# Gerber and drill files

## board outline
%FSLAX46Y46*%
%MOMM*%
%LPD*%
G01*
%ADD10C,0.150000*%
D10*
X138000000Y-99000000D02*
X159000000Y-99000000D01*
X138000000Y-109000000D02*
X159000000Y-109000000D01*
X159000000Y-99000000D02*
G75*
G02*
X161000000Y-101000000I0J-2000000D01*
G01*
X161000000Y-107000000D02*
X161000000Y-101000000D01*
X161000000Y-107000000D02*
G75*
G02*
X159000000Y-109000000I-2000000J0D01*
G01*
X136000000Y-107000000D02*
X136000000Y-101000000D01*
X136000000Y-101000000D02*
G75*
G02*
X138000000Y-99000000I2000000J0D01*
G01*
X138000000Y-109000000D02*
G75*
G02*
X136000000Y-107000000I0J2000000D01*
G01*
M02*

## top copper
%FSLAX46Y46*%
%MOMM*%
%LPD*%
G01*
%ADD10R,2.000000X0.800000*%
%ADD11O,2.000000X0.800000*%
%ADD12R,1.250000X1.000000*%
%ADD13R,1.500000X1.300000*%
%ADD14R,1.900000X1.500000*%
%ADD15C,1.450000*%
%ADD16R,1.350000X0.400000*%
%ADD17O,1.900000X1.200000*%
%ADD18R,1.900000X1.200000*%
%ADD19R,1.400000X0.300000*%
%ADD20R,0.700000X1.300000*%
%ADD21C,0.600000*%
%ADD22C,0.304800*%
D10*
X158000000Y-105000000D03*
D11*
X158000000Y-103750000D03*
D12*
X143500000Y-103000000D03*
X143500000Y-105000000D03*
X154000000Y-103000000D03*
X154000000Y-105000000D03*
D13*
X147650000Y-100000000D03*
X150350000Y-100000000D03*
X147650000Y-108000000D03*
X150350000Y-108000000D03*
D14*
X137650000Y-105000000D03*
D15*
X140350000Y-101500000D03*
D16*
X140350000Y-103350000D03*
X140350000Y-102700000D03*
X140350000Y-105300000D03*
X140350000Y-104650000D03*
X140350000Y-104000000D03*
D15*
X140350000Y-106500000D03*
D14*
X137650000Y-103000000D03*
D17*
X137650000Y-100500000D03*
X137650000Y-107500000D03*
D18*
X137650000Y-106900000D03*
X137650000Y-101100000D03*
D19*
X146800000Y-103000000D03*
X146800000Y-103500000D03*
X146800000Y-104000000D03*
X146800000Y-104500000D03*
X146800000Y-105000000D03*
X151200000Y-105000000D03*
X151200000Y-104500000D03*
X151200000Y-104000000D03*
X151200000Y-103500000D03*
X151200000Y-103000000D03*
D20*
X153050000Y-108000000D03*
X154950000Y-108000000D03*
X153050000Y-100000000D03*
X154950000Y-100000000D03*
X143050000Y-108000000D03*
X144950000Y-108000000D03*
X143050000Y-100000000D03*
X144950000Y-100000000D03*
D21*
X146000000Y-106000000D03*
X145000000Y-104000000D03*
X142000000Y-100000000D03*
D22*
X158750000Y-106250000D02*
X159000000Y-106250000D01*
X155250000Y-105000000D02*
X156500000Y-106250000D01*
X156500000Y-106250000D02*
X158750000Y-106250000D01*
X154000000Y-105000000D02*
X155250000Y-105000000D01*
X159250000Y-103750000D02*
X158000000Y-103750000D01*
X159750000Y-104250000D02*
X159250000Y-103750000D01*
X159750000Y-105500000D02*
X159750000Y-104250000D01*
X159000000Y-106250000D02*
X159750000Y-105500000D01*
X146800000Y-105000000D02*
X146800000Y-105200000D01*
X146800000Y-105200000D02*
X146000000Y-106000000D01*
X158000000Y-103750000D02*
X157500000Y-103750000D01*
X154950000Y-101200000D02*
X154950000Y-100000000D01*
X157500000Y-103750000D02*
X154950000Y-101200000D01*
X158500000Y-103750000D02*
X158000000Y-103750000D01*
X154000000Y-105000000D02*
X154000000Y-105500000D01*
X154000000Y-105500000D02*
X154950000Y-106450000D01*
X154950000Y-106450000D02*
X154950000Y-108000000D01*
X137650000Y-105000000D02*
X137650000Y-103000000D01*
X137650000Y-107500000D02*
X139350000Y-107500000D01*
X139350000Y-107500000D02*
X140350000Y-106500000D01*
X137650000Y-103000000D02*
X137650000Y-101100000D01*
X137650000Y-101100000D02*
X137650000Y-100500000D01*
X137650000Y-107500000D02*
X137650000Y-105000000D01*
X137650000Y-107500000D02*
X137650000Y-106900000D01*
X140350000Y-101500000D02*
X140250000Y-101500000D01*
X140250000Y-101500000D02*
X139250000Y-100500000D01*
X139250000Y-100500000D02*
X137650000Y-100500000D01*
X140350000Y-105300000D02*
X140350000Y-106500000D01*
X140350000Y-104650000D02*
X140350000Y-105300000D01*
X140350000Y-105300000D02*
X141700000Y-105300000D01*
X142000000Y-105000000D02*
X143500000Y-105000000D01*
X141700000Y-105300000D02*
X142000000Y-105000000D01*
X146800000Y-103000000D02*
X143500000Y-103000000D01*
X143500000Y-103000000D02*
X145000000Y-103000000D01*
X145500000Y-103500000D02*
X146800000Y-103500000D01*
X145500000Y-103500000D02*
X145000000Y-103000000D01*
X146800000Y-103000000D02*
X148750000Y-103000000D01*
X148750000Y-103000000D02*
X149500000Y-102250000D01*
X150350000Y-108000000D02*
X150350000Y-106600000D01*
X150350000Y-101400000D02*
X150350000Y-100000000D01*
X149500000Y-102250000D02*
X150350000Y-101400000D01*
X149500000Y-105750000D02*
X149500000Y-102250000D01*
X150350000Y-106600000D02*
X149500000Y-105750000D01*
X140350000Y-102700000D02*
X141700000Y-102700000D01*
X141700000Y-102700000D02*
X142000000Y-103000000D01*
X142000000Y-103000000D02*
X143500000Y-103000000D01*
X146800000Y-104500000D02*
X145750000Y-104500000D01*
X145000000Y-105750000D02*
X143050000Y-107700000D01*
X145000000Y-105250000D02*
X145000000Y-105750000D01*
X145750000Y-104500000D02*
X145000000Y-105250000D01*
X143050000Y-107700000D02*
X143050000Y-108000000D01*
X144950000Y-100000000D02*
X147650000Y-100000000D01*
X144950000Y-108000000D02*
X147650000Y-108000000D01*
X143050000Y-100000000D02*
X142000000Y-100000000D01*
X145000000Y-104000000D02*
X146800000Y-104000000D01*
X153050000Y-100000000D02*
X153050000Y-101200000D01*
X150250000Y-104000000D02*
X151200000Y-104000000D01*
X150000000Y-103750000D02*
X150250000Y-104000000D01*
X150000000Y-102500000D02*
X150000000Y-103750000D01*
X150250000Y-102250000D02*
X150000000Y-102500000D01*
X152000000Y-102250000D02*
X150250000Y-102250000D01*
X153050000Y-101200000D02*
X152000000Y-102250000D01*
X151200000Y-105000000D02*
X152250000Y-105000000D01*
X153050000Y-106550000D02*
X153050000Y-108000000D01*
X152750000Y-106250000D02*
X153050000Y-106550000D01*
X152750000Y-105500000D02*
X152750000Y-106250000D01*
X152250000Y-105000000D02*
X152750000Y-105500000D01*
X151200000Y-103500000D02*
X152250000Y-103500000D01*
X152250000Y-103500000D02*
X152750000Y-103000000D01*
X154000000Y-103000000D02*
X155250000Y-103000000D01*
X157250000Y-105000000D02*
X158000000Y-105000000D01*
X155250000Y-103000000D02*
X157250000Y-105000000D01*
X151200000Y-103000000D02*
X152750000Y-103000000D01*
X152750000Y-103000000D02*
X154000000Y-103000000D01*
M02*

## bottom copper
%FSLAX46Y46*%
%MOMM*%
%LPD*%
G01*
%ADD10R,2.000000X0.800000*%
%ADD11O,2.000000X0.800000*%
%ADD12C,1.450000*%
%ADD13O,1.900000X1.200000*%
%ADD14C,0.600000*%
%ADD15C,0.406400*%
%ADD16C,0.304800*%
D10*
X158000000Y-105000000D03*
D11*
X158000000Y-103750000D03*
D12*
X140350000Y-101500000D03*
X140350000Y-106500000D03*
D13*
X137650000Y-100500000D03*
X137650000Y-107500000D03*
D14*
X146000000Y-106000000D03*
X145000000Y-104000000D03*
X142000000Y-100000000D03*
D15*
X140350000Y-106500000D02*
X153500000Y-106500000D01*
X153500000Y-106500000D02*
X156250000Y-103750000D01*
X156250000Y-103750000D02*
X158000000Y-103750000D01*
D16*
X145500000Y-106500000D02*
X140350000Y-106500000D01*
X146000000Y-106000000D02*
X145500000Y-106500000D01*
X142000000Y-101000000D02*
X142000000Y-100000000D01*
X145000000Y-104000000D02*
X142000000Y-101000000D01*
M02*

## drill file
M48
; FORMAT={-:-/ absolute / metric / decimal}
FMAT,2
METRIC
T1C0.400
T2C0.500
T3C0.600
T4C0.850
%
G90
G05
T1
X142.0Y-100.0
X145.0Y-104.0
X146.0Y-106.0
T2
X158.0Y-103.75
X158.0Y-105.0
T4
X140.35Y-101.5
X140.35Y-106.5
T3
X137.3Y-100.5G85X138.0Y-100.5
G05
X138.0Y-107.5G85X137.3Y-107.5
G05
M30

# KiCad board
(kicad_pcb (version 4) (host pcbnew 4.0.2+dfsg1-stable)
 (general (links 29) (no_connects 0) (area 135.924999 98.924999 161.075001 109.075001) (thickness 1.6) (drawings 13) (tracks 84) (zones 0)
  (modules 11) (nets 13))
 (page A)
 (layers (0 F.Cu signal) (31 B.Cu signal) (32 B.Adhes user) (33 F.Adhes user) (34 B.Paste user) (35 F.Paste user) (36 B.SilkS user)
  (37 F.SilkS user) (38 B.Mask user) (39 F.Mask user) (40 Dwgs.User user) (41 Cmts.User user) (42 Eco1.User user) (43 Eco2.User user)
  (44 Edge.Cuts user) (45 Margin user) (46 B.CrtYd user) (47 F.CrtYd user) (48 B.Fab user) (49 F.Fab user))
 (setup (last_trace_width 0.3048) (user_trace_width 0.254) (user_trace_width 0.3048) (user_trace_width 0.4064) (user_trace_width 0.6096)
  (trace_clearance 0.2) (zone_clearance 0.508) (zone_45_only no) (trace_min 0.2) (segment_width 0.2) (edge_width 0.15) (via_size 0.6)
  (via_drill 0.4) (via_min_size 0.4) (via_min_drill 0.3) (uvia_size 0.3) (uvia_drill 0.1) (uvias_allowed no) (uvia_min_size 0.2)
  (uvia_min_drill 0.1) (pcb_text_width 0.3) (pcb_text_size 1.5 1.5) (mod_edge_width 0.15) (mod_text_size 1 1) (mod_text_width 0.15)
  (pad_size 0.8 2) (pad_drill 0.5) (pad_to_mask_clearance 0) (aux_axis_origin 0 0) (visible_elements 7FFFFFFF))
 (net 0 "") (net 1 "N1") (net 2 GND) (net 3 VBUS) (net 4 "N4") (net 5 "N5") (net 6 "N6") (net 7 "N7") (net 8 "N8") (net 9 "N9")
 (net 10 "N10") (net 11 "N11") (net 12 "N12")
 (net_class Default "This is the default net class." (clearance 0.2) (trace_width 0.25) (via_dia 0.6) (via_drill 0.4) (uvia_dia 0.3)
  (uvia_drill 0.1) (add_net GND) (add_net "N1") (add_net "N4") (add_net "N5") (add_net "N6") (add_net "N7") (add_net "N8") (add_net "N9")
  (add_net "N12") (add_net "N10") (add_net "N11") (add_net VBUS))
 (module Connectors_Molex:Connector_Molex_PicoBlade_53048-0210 (layer F.Cu) (at 158 105 90)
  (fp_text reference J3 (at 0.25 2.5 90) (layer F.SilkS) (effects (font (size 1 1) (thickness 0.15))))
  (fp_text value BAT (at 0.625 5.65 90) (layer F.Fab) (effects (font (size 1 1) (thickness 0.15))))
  (pad 1 thru_hole rect (at 0 0 90) (size 0.8 2) (drill 0.5) (layers *.Cu *.Mask F.SilkS) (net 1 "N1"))
  (pad 2 thru_hole oval (at 1.25 0 90) (size 0.8 2) (drill 0.5) (layers *.Cu *.Mask F.SilkS) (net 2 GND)))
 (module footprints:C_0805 (layer F.Cu) (at 143.5 104 270)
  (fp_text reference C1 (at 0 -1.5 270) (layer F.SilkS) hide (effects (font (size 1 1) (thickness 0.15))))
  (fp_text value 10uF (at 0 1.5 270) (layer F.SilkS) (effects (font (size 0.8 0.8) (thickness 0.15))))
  (pad 1 smd rect (at -1 0 270) (size 1 1.25) (layers F.Cu F.Paste F.Mask) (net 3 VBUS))
  (pad 2 smd rect (at 1 0 270) (size 1 1.25) (layers F.Cu F.Paste F.Mask) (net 2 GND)))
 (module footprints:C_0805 (layer F.Cu) (at 154 104 270)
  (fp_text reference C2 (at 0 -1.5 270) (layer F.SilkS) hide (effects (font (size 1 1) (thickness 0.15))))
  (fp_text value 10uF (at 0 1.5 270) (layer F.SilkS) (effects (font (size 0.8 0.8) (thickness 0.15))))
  (pad 1 smd rect (at -1 0 270) (size 1 1.25) (layers F.Cu F.Paste F.Mask) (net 1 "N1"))
  (pad 2 smd rect (at 1 0 270) (size 1 1.25) (layers F.Cu F.Paste F.Mask) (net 2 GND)))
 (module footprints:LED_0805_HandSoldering (layer F.Cu) (at 149 100)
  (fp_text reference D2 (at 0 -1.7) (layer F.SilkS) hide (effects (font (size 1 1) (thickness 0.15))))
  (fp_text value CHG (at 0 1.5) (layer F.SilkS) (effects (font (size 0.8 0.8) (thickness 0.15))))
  (pad 1 smd rect (at -1.35 0) (size 1.5 1.3) (layers F.Cu F.Paste F.Mask) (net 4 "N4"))
  (pad 2 smd rect (at 1.35 0) (size 1.5 1.3) (layers F.Cu F.Paste F.Mask) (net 3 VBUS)))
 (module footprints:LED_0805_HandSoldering (layer F.Cu) (at 149 108)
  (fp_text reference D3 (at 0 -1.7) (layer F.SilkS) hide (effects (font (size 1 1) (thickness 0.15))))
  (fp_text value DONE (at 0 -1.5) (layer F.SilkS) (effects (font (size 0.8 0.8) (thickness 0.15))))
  (pad 1 smd rect (at -1.35 0) (size 1.5 1.3) (layers F.Cu F.Paste F.Mask) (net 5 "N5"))
  (pad 2 smd rect (at 1.35 0) (size 1.5 1.3) (layers F.Cu F.Paste F.Mask) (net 3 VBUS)))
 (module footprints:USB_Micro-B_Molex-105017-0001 (layer F.Cu) (at 138 104 270)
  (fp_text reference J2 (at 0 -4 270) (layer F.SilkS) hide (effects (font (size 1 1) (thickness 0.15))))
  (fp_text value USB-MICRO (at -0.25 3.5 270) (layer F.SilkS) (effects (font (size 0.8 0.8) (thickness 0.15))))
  (pad 5 smd rect (at 1 0.35 270) (size 1.5 1.9) (layers F.Cu F.Paste F.Mask) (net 2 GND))
  (pad 5 thru_hole circle (at -2.5 -2.35 270) (size 1.45 1.45) (drill 0.85) (layers *.Cu *.Mask) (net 2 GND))
  (pad 2 smd rect (at -0.65 -2.35 270) (size 0.4 1.35) (layers F.Cu F.Paste F.Mask) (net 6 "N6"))
  (pad 1 smd rect (at -1.3 -2.35 270) (size 0.4 1.35) (layers F.Cu F.Paste F.Mask) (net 3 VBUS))
  (pad 5 smd rect (at 1.3 -2.35 270) (size 0.4 1.35) (layers F.Cu F.Paste F.Mask) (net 2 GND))
  (pad 4 smd rect (at 0.65 -2.35 270) (size 0.4 1.35) (layers F.Cu F.Paste F.Mask) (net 2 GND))
  (pad 3 smd rect (at 0 -2.35 270) (size 0.4 1.35) (layers F.Cu F.Paste F.Mask) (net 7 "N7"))
  (pad 5 thru_hole circle (at 2.5 -2.35 270) (size 1.45 1.45) (drill 0.85) (layers *.Cu *.Mask) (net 2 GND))
  (pad 5 smd rect (at -1 0.35 270) (size 1.5 1.9) (layers F.Cu F.Paste F.Mask) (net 2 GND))
  (pad 5 thru_hole oval (at -3.5 0.35 90) (size 1.2 1.9) (drill oval 0.6 1.3) (layers *.Cu *.Mask) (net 2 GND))
  (pad 5 thru_hole oval (at 3.5 0.35 270) (size 1.2 1.9) (drill oval 0.6 1.3) (layers *.Cu *.Mask) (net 2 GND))
  (pad 5 smd rect (at 2.9 0.35 270) (size 1.2 1.9) (layers F.Cu F.Mask) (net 2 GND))
  (pad 5 smd rect (at -2.9 0.35 270) (size 1.2 1.9) (layers F.Cu F.Mask) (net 2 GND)))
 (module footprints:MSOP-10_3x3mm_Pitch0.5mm (layer F.Cu) (at 149 104)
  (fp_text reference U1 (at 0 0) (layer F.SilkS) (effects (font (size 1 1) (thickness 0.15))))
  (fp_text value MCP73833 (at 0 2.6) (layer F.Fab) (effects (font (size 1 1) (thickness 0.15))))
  (pad 1 smd rect (at -2.2 -1) (size 1.4 0.3) (layers F.Cu F.Paste F.Mask) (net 3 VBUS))
  (pad 2 smd rect (at -2.2 -0.5) (size 1.4 0.3) (layers F.Cu F.Paste F.Mask) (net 3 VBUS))
  (pad 3 smd rect (at -2.2 0) (size 1.4 0.3) (layers F.Cu F.Paste F.Mask) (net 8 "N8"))
  (pad 4 smd rect (at -2.2 0.5) (size 1.4 0.3) (layers F.Cu F.Paste F.Mask) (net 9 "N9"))
  (pad 5 smd rect (at -2.2 1) (size 1.4 0.3) (layers F.Cu F.Paste F.Mask) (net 2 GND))
  (pad 6 smd rect (at 2.2 1) (size 1.4 0.3) (layers F.Cu F.Paste F.Mask) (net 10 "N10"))
  (pad 7 smd rect (at 2.2 0.5) (size 1.4 0.3) (layers F.Cu F.Paste F.Mask) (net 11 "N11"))
  (pad 8 smd rect (at 2.2 0) (size 1.4 0.3) (layers F.Cu F.Paste F.Mask) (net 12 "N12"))
  (pad 9 smd rect (at 2.2 -0.5) (size 1.4 0.3) (layers F.Cu F.Paste F.Mask) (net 1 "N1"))
  (pad 10 smd rect (at 2.2 -1) (size 1.4 0.3) (layers F.Cu F.Paste F.Mask) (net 1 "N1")))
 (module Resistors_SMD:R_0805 (layer F.Cu) (at 154 108)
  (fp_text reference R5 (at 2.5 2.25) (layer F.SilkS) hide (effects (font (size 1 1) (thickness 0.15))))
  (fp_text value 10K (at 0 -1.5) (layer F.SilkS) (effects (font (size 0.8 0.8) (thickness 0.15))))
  (pad 1 smd rect (at -0.95 0) (size 0.7 1.3) (layers F.Cu F.Paste F.Mask) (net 10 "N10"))
  (pad 2 smd rect (at 0.95 0) (size 0.7 1.3) (layers F.Cu F.Paste F.Mask) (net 2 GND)))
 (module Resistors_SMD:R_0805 (layer F.Cu) (at 154 100)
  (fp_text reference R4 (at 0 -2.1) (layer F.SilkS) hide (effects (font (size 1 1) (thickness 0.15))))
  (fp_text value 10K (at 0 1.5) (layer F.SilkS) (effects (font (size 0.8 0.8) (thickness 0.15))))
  (pad 1 smd rect (at -0.95 0) (size 0.7 1.3) (layers F.Cu F.Paste F.Mask) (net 12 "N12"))
  (pad 2 smd rect (at 0.95 0) (size 0.7 1.3) (layers F.Cu F.Paste F.Mask) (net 2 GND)))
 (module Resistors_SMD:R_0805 (layer F.Cu) (at 144 108)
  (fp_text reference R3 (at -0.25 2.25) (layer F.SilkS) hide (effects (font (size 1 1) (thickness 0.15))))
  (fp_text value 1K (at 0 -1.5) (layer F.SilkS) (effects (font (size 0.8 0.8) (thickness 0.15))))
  (pad 1 smd rect (at -0.95 0) (size 0.7 1.3) (layers F.Cu F.Paste F.Mask) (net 9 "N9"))
  (pad 2 smd rect (at 0.95 0) (size 0.7 1.3) (layers F.Cu F.Paste F.Mask) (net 5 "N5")))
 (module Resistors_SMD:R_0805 (layer F.Cu) (at 144 100)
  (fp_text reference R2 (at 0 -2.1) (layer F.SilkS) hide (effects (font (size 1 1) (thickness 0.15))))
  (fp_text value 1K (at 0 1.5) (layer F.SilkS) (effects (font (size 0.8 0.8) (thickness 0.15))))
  (pad 1 smd rect (at -0.95 0) (size 0.7 1.3) (layers F.Cu F.Paste F.Mask) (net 8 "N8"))
  (pad 2 smd rect (at 0.95 0) (size 0.7 1.3) (layers F.Cu F.Paste F.Mask) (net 4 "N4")))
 (gr_line (start 138 99) (end 159 99) (angle 90) (layer Edge.Cuts) (width 0.15))
 (gr_line (start 138 109) (end 159 109) (angle 90) (layer Edge.Cuts) (width 0.15))
 (gr_arc (start 159 101) (end 159 99) (angle 90) (layer Edge.Cuts) (width 0.15))
 (gr_line (start 161 107) (end 161 101) (angle 90) (layer Edge.Cuts) (width 0.15))
 (gr_arc (start 159 107) (end 161 107) (angle 90) (layer Edge.Cuts) (width 0.15))
 (gr_line (start 136 107) (end 136 101) (angle 90) (layer Edge.Cuts) (width 0.15))
 (gr_arc (start 138 101) (end 136 101) (angle 90) (layer Edge.Cuts) (width 0.15))
 (gr_arc (start 138 107) (end 138 109) (angle 90) (layer Edge.Cuts) (width 0.15))
 (segment (start 158.75 106.25) (end 159 106.25) (width 0.3048) (layer F.Cu) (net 2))
 (segment (start 155.25 105) (end 156.5 106.25) (width 0.3048) (layer F.Cu) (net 2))
 (segment (start 156.5 106.25) (end 158.75 106.25) (width 0.3048) (layer F.Cu) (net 2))
 (segment (start 154 105) (end 155.25 105) (width 0.3048) (layer F.Cu) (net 2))
 (segment (start 159.25 103.75) (end 158 103.75) (width 0.3048) (layer F.Cu) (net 2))
 (segment (start 159.75 104.25) (end 159.25 103.75) (width 0.3048) (layer F.Cu) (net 2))
 (segment (start 159.75 105.5) (end 159.75 104.25) (width 0.3048) (layer F.Cu) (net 2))
 (segment (start 159 106.25) (end 159.75 105.5) (width 0.3048) (layer F.Cu) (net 2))
 (segment (start 140.35 106.5) (end 153.5 106.5) (width 0.4064) (layer B.Cu) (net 2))
 (segment (start 153.5 106.5) (end 156.25 103.75) (width 0.4064) (layer B.Cu) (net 2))
 (segment (start 156.25 103.75) (end 158 103.75) (width 0.4064) (layer B.Cu) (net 2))
 (segment (start 146.8 105) (end 146.8 105.2) (width 0.3048) (layer F.Cu) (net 2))
 (segment (start 145.5 106.5) (end 140.35 106.5) (width 0.3048) (layer B.Cu) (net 2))
 (segment (start 146 106) (end 145.5 106.5) (width 0.3048) (layer B.Cu) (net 2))
 (via (at 146 106) (size 0.6) (drill 0.4) (layers F.Cu B.Cu) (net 2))
 (segment (start 146.8 105.2) (end 146 106) (width 0.3048) (layer F.Cu) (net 2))
 (segment (start 158 103.75) (end 157.5 103.75) (width 0.3048) (layer F.Cu) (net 2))
 (segment (start 154.95 101.2) (end 154.95 100) (width 0.3048) (layer F.Cu) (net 2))
 (segment (start 157.5 103.75) (end 154.95 101.2) (width 0.3048) (layer F.Cu) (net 2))
 (segment (start 158.5 103.75) (end 158 103.75) (width 0.3048) (layer F.Cu) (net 2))
 (segment (start 154 105) (end 154 105.5) (width 0.3048) (layer F.Cu) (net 2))
 (segment (start 154 105.5) (end 154.95 106.45) (width 0.3048) (layer F.Cu) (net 2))
 (segment (start 154.95 106.45) (end 154.95 108) (width 0.3048) (layer F.Cu) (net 2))
 (segment (start 137.65 105) (end 137.65 103) (width 0.3048) (layer F.Cu) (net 2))
 (segment (start 137.65 107.5) (end 139.35 107.5) (width 0.3048) (layer F.Cu) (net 2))
 (segment (start 139.35 107.5) (end 140.35 106.5) (width 0.3048) (layer F.Cu) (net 2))
 (segment (start 137.65 103) (end 137.65 101.1) (width 0.3048) (layer F.Cu) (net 2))
 (segment (start 137.65 101.1) (end 137.65 100.5) (width 0.3048) (layer F.Cu) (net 2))
 (segment (start 137.65 107.5) (end 137.65 105) (width 0.3048) (layer F.Cu) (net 2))
 (segment (start 137.65 107.5) (end 137.65 106.9) (width 0.3048) (layer F.Cu) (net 2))
 (segment (start 140.35 101.5) (end 140.25 101.5) (width 0.3048) (layer F.Cu) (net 2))
 (segment (start 140.25 101.5) (end 139.25 100.5) (width 0.3048) (layer F.Cu) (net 2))
 (segment (start 139.25 100.5) (end 137.65 100.5) (width 0.3048) (layer F.Cu) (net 2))
 (segment (start 140.35 105.3) (end 140.35 106.5) (width 0.3048) (layer F.Cu) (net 2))
 (segment (start 140.35 104.65) (end 140.35 105.3) (width 0.3048) (layer F.Cu) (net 2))
 (segment (start 140.35 105.3) (end 141.7 105.3) (width 0.3048) (layer F.Cu) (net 2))
 (segment (start 142 105) (end 143.5 105) (width 0.3048) (layer F.Cu) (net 2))
 (segment (start 141.7 105.3) (end 142 105) (width 0.3048) (layer F.Cu) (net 2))
 (segment (start 146.8 103) (end 143.5 103) (width 0.3048) (layer F.Cu) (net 3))
 (segment (start 143.5 103) (end 145 103) (width 0.3048) (layer F.Cu) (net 3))
 (segment (start 145.5 103.5) (end 146.8 103.5) (width 0.3048) (layer F.Cu) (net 3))
 (segment (start 145.5 103.5) (end 145 103) (width 0.3048) (layer F.Cu) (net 3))
 (segment (start 146.8 103) (end 148.75 103) (width 0.3048) (layer F.Cu) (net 3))
 (segment (start 148.75 103) (end 149.5 102.25) (width 0.3048) (layer F.Cu) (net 3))
 (segment (start 150.35 108) (end 150.35 106.6) (width 0.3048) (layer F.Cu) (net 3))
 (segment (start 150.35 101.4) (end 150.35 100) (width 0.3048) (layer F.Cu) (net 3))
 (segment (start 149.5 102.25) (end 150.35 101.4) (width 0.3048) (layer F.Cu) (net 3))
 (segment (start 149.5 105.75) (end 149.5 102.25) (width 0.3048) (layer F.Cu) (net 3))
 (segment (start 150.35 106.6) (end 149.5 105.75) (width 0.3048) (layer F.Cu) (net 3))
 (segment (start 140.35 102.7) (end 141.7 102.7) (width 0.3048) (layer F.Cu) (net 3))
 (segment (start 141.7 102.7) (end 142 103) (width 0.3048) (layer F.Cu) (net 3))
 (segment (start 142 103) (end 143.5 103) (width 0.3048) (layer F.Cu) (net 3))
 (segment (start 146.8 104.5) (end 145.75 104.5) (width 0.3048) (layer F.Cu) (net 9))
 (segment (start 145 105.75) (end 143.05 107.7) (width 0.3048) (layer F.Cu) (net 9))
 (segment (start 145 105.25) (end 145 105.75) (width 0.3048) (layer F.Cu) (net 9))
 (segment (start 145.75 104.5) (end 145 105.25) (width 0.3048) (layer F.Cu) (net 9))
 (segment (start 143.05 107.7) (end 143.05 108) (width 0.3048) (layer F.Cu) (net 9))
 (segment (start 144.95 100) (end 147.65 100) (width 0.3048) (layer F.Cu) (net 4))
 (segment (start 144.95 108) (end 147.65 108) (width 0.3048) (layer F.Cu) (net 5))
 (via (at 145 104) (size 0.6) (drill 0.4) (layers F.Cu B.Cu) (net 8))
 (segment (start 142 101) (end 142 100) (width 0.3048) (layer B.Cu) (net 8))
 (via (at 142 100) (size 0.6) (drill 0.4) (layers F.Cu B.Cu) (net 8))
 (segment (start 143.05 100) (end 142 100) (width 0.3048) (layer F.Cu) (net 8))
 (segment (start 145 104) (end 146.8 104) (width 0.3048) (layer F.Cu) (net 8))
 (segment (start 145 104) (end 142 101) (width 0.3048) (layer B.Cu) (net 8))
 (segment (start 153.05 100) (end 153.05 101.2) (width 0.3048) (layer F.Cu) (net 12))
 (segment (start 150.25 104) (end 151.2 104) (width 0.3048) (layer F.Cu) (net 12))
 (segment (start 150 103.75) (end 150.25 104) (width 0.3048) (layer F.Cu) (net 12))
 (segment (start 150 102.5) (end 150 103.75) (width 0.3048) (layer F.Cu) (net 12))
 (segment (start 150.25 102.25) (end 150 102.5) (width 0.3048) (layer F.Cu) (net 12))
 (segment (start 152 102.25) (end 150.25 102.25) (width 0.3048) (layer F.Cu) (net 12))
 (segment (start 153.05 101.2) (end 152 102.25) (width 0.3048) (layer F.Cu) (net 12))
 (segment (start 151.2 105) (end 152.25 105) (width 0.3048) (layer F.Cu) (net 10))
 (segment (start 153.05 106.55) (end 153.05 108) (width 0.3048) (layer F.Cu) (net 10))
 (segment (start 152.75 106.25) (end 153.05 106.55) (width 0.3048) (layer F.Cu) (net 10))
 (segment (start 152.75 105.5) (end 152.75 106.25) (width 0.3048) (layer F.Cu) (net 10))
 (segment (start 152.25 105) (end 152.75 105.5) (width 0.3048) (layer F.Cu) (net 10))
 (segment (start 151.2 103.5) (end 152.25 103.5) (width 0.3048) (layer F.Cu) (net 1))
 (segment (start 152.25 103.5) (end 152.75 103) (width 0.3048) (layer F.Cu) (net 1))
 (segment (start 154 103) (end 155.25 103) (width 0.3048) (layer F.Cu) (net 1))
 (segment (start 157.25 105) (end 158 105) (width 0.3048) (layer F.Cu) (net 1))
 (segment (start 155.25 103) (end 157.25 105) (width 0.3048) (layer F.Cu) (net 1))
 (segment (start 151.2 103) (end 152.75 103) (width 0.3048) (layer F.Cu) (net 1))
 (segment (start 152.75 103) (end 154 103) (width 0.3048) (layer F.Cu) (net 1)))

